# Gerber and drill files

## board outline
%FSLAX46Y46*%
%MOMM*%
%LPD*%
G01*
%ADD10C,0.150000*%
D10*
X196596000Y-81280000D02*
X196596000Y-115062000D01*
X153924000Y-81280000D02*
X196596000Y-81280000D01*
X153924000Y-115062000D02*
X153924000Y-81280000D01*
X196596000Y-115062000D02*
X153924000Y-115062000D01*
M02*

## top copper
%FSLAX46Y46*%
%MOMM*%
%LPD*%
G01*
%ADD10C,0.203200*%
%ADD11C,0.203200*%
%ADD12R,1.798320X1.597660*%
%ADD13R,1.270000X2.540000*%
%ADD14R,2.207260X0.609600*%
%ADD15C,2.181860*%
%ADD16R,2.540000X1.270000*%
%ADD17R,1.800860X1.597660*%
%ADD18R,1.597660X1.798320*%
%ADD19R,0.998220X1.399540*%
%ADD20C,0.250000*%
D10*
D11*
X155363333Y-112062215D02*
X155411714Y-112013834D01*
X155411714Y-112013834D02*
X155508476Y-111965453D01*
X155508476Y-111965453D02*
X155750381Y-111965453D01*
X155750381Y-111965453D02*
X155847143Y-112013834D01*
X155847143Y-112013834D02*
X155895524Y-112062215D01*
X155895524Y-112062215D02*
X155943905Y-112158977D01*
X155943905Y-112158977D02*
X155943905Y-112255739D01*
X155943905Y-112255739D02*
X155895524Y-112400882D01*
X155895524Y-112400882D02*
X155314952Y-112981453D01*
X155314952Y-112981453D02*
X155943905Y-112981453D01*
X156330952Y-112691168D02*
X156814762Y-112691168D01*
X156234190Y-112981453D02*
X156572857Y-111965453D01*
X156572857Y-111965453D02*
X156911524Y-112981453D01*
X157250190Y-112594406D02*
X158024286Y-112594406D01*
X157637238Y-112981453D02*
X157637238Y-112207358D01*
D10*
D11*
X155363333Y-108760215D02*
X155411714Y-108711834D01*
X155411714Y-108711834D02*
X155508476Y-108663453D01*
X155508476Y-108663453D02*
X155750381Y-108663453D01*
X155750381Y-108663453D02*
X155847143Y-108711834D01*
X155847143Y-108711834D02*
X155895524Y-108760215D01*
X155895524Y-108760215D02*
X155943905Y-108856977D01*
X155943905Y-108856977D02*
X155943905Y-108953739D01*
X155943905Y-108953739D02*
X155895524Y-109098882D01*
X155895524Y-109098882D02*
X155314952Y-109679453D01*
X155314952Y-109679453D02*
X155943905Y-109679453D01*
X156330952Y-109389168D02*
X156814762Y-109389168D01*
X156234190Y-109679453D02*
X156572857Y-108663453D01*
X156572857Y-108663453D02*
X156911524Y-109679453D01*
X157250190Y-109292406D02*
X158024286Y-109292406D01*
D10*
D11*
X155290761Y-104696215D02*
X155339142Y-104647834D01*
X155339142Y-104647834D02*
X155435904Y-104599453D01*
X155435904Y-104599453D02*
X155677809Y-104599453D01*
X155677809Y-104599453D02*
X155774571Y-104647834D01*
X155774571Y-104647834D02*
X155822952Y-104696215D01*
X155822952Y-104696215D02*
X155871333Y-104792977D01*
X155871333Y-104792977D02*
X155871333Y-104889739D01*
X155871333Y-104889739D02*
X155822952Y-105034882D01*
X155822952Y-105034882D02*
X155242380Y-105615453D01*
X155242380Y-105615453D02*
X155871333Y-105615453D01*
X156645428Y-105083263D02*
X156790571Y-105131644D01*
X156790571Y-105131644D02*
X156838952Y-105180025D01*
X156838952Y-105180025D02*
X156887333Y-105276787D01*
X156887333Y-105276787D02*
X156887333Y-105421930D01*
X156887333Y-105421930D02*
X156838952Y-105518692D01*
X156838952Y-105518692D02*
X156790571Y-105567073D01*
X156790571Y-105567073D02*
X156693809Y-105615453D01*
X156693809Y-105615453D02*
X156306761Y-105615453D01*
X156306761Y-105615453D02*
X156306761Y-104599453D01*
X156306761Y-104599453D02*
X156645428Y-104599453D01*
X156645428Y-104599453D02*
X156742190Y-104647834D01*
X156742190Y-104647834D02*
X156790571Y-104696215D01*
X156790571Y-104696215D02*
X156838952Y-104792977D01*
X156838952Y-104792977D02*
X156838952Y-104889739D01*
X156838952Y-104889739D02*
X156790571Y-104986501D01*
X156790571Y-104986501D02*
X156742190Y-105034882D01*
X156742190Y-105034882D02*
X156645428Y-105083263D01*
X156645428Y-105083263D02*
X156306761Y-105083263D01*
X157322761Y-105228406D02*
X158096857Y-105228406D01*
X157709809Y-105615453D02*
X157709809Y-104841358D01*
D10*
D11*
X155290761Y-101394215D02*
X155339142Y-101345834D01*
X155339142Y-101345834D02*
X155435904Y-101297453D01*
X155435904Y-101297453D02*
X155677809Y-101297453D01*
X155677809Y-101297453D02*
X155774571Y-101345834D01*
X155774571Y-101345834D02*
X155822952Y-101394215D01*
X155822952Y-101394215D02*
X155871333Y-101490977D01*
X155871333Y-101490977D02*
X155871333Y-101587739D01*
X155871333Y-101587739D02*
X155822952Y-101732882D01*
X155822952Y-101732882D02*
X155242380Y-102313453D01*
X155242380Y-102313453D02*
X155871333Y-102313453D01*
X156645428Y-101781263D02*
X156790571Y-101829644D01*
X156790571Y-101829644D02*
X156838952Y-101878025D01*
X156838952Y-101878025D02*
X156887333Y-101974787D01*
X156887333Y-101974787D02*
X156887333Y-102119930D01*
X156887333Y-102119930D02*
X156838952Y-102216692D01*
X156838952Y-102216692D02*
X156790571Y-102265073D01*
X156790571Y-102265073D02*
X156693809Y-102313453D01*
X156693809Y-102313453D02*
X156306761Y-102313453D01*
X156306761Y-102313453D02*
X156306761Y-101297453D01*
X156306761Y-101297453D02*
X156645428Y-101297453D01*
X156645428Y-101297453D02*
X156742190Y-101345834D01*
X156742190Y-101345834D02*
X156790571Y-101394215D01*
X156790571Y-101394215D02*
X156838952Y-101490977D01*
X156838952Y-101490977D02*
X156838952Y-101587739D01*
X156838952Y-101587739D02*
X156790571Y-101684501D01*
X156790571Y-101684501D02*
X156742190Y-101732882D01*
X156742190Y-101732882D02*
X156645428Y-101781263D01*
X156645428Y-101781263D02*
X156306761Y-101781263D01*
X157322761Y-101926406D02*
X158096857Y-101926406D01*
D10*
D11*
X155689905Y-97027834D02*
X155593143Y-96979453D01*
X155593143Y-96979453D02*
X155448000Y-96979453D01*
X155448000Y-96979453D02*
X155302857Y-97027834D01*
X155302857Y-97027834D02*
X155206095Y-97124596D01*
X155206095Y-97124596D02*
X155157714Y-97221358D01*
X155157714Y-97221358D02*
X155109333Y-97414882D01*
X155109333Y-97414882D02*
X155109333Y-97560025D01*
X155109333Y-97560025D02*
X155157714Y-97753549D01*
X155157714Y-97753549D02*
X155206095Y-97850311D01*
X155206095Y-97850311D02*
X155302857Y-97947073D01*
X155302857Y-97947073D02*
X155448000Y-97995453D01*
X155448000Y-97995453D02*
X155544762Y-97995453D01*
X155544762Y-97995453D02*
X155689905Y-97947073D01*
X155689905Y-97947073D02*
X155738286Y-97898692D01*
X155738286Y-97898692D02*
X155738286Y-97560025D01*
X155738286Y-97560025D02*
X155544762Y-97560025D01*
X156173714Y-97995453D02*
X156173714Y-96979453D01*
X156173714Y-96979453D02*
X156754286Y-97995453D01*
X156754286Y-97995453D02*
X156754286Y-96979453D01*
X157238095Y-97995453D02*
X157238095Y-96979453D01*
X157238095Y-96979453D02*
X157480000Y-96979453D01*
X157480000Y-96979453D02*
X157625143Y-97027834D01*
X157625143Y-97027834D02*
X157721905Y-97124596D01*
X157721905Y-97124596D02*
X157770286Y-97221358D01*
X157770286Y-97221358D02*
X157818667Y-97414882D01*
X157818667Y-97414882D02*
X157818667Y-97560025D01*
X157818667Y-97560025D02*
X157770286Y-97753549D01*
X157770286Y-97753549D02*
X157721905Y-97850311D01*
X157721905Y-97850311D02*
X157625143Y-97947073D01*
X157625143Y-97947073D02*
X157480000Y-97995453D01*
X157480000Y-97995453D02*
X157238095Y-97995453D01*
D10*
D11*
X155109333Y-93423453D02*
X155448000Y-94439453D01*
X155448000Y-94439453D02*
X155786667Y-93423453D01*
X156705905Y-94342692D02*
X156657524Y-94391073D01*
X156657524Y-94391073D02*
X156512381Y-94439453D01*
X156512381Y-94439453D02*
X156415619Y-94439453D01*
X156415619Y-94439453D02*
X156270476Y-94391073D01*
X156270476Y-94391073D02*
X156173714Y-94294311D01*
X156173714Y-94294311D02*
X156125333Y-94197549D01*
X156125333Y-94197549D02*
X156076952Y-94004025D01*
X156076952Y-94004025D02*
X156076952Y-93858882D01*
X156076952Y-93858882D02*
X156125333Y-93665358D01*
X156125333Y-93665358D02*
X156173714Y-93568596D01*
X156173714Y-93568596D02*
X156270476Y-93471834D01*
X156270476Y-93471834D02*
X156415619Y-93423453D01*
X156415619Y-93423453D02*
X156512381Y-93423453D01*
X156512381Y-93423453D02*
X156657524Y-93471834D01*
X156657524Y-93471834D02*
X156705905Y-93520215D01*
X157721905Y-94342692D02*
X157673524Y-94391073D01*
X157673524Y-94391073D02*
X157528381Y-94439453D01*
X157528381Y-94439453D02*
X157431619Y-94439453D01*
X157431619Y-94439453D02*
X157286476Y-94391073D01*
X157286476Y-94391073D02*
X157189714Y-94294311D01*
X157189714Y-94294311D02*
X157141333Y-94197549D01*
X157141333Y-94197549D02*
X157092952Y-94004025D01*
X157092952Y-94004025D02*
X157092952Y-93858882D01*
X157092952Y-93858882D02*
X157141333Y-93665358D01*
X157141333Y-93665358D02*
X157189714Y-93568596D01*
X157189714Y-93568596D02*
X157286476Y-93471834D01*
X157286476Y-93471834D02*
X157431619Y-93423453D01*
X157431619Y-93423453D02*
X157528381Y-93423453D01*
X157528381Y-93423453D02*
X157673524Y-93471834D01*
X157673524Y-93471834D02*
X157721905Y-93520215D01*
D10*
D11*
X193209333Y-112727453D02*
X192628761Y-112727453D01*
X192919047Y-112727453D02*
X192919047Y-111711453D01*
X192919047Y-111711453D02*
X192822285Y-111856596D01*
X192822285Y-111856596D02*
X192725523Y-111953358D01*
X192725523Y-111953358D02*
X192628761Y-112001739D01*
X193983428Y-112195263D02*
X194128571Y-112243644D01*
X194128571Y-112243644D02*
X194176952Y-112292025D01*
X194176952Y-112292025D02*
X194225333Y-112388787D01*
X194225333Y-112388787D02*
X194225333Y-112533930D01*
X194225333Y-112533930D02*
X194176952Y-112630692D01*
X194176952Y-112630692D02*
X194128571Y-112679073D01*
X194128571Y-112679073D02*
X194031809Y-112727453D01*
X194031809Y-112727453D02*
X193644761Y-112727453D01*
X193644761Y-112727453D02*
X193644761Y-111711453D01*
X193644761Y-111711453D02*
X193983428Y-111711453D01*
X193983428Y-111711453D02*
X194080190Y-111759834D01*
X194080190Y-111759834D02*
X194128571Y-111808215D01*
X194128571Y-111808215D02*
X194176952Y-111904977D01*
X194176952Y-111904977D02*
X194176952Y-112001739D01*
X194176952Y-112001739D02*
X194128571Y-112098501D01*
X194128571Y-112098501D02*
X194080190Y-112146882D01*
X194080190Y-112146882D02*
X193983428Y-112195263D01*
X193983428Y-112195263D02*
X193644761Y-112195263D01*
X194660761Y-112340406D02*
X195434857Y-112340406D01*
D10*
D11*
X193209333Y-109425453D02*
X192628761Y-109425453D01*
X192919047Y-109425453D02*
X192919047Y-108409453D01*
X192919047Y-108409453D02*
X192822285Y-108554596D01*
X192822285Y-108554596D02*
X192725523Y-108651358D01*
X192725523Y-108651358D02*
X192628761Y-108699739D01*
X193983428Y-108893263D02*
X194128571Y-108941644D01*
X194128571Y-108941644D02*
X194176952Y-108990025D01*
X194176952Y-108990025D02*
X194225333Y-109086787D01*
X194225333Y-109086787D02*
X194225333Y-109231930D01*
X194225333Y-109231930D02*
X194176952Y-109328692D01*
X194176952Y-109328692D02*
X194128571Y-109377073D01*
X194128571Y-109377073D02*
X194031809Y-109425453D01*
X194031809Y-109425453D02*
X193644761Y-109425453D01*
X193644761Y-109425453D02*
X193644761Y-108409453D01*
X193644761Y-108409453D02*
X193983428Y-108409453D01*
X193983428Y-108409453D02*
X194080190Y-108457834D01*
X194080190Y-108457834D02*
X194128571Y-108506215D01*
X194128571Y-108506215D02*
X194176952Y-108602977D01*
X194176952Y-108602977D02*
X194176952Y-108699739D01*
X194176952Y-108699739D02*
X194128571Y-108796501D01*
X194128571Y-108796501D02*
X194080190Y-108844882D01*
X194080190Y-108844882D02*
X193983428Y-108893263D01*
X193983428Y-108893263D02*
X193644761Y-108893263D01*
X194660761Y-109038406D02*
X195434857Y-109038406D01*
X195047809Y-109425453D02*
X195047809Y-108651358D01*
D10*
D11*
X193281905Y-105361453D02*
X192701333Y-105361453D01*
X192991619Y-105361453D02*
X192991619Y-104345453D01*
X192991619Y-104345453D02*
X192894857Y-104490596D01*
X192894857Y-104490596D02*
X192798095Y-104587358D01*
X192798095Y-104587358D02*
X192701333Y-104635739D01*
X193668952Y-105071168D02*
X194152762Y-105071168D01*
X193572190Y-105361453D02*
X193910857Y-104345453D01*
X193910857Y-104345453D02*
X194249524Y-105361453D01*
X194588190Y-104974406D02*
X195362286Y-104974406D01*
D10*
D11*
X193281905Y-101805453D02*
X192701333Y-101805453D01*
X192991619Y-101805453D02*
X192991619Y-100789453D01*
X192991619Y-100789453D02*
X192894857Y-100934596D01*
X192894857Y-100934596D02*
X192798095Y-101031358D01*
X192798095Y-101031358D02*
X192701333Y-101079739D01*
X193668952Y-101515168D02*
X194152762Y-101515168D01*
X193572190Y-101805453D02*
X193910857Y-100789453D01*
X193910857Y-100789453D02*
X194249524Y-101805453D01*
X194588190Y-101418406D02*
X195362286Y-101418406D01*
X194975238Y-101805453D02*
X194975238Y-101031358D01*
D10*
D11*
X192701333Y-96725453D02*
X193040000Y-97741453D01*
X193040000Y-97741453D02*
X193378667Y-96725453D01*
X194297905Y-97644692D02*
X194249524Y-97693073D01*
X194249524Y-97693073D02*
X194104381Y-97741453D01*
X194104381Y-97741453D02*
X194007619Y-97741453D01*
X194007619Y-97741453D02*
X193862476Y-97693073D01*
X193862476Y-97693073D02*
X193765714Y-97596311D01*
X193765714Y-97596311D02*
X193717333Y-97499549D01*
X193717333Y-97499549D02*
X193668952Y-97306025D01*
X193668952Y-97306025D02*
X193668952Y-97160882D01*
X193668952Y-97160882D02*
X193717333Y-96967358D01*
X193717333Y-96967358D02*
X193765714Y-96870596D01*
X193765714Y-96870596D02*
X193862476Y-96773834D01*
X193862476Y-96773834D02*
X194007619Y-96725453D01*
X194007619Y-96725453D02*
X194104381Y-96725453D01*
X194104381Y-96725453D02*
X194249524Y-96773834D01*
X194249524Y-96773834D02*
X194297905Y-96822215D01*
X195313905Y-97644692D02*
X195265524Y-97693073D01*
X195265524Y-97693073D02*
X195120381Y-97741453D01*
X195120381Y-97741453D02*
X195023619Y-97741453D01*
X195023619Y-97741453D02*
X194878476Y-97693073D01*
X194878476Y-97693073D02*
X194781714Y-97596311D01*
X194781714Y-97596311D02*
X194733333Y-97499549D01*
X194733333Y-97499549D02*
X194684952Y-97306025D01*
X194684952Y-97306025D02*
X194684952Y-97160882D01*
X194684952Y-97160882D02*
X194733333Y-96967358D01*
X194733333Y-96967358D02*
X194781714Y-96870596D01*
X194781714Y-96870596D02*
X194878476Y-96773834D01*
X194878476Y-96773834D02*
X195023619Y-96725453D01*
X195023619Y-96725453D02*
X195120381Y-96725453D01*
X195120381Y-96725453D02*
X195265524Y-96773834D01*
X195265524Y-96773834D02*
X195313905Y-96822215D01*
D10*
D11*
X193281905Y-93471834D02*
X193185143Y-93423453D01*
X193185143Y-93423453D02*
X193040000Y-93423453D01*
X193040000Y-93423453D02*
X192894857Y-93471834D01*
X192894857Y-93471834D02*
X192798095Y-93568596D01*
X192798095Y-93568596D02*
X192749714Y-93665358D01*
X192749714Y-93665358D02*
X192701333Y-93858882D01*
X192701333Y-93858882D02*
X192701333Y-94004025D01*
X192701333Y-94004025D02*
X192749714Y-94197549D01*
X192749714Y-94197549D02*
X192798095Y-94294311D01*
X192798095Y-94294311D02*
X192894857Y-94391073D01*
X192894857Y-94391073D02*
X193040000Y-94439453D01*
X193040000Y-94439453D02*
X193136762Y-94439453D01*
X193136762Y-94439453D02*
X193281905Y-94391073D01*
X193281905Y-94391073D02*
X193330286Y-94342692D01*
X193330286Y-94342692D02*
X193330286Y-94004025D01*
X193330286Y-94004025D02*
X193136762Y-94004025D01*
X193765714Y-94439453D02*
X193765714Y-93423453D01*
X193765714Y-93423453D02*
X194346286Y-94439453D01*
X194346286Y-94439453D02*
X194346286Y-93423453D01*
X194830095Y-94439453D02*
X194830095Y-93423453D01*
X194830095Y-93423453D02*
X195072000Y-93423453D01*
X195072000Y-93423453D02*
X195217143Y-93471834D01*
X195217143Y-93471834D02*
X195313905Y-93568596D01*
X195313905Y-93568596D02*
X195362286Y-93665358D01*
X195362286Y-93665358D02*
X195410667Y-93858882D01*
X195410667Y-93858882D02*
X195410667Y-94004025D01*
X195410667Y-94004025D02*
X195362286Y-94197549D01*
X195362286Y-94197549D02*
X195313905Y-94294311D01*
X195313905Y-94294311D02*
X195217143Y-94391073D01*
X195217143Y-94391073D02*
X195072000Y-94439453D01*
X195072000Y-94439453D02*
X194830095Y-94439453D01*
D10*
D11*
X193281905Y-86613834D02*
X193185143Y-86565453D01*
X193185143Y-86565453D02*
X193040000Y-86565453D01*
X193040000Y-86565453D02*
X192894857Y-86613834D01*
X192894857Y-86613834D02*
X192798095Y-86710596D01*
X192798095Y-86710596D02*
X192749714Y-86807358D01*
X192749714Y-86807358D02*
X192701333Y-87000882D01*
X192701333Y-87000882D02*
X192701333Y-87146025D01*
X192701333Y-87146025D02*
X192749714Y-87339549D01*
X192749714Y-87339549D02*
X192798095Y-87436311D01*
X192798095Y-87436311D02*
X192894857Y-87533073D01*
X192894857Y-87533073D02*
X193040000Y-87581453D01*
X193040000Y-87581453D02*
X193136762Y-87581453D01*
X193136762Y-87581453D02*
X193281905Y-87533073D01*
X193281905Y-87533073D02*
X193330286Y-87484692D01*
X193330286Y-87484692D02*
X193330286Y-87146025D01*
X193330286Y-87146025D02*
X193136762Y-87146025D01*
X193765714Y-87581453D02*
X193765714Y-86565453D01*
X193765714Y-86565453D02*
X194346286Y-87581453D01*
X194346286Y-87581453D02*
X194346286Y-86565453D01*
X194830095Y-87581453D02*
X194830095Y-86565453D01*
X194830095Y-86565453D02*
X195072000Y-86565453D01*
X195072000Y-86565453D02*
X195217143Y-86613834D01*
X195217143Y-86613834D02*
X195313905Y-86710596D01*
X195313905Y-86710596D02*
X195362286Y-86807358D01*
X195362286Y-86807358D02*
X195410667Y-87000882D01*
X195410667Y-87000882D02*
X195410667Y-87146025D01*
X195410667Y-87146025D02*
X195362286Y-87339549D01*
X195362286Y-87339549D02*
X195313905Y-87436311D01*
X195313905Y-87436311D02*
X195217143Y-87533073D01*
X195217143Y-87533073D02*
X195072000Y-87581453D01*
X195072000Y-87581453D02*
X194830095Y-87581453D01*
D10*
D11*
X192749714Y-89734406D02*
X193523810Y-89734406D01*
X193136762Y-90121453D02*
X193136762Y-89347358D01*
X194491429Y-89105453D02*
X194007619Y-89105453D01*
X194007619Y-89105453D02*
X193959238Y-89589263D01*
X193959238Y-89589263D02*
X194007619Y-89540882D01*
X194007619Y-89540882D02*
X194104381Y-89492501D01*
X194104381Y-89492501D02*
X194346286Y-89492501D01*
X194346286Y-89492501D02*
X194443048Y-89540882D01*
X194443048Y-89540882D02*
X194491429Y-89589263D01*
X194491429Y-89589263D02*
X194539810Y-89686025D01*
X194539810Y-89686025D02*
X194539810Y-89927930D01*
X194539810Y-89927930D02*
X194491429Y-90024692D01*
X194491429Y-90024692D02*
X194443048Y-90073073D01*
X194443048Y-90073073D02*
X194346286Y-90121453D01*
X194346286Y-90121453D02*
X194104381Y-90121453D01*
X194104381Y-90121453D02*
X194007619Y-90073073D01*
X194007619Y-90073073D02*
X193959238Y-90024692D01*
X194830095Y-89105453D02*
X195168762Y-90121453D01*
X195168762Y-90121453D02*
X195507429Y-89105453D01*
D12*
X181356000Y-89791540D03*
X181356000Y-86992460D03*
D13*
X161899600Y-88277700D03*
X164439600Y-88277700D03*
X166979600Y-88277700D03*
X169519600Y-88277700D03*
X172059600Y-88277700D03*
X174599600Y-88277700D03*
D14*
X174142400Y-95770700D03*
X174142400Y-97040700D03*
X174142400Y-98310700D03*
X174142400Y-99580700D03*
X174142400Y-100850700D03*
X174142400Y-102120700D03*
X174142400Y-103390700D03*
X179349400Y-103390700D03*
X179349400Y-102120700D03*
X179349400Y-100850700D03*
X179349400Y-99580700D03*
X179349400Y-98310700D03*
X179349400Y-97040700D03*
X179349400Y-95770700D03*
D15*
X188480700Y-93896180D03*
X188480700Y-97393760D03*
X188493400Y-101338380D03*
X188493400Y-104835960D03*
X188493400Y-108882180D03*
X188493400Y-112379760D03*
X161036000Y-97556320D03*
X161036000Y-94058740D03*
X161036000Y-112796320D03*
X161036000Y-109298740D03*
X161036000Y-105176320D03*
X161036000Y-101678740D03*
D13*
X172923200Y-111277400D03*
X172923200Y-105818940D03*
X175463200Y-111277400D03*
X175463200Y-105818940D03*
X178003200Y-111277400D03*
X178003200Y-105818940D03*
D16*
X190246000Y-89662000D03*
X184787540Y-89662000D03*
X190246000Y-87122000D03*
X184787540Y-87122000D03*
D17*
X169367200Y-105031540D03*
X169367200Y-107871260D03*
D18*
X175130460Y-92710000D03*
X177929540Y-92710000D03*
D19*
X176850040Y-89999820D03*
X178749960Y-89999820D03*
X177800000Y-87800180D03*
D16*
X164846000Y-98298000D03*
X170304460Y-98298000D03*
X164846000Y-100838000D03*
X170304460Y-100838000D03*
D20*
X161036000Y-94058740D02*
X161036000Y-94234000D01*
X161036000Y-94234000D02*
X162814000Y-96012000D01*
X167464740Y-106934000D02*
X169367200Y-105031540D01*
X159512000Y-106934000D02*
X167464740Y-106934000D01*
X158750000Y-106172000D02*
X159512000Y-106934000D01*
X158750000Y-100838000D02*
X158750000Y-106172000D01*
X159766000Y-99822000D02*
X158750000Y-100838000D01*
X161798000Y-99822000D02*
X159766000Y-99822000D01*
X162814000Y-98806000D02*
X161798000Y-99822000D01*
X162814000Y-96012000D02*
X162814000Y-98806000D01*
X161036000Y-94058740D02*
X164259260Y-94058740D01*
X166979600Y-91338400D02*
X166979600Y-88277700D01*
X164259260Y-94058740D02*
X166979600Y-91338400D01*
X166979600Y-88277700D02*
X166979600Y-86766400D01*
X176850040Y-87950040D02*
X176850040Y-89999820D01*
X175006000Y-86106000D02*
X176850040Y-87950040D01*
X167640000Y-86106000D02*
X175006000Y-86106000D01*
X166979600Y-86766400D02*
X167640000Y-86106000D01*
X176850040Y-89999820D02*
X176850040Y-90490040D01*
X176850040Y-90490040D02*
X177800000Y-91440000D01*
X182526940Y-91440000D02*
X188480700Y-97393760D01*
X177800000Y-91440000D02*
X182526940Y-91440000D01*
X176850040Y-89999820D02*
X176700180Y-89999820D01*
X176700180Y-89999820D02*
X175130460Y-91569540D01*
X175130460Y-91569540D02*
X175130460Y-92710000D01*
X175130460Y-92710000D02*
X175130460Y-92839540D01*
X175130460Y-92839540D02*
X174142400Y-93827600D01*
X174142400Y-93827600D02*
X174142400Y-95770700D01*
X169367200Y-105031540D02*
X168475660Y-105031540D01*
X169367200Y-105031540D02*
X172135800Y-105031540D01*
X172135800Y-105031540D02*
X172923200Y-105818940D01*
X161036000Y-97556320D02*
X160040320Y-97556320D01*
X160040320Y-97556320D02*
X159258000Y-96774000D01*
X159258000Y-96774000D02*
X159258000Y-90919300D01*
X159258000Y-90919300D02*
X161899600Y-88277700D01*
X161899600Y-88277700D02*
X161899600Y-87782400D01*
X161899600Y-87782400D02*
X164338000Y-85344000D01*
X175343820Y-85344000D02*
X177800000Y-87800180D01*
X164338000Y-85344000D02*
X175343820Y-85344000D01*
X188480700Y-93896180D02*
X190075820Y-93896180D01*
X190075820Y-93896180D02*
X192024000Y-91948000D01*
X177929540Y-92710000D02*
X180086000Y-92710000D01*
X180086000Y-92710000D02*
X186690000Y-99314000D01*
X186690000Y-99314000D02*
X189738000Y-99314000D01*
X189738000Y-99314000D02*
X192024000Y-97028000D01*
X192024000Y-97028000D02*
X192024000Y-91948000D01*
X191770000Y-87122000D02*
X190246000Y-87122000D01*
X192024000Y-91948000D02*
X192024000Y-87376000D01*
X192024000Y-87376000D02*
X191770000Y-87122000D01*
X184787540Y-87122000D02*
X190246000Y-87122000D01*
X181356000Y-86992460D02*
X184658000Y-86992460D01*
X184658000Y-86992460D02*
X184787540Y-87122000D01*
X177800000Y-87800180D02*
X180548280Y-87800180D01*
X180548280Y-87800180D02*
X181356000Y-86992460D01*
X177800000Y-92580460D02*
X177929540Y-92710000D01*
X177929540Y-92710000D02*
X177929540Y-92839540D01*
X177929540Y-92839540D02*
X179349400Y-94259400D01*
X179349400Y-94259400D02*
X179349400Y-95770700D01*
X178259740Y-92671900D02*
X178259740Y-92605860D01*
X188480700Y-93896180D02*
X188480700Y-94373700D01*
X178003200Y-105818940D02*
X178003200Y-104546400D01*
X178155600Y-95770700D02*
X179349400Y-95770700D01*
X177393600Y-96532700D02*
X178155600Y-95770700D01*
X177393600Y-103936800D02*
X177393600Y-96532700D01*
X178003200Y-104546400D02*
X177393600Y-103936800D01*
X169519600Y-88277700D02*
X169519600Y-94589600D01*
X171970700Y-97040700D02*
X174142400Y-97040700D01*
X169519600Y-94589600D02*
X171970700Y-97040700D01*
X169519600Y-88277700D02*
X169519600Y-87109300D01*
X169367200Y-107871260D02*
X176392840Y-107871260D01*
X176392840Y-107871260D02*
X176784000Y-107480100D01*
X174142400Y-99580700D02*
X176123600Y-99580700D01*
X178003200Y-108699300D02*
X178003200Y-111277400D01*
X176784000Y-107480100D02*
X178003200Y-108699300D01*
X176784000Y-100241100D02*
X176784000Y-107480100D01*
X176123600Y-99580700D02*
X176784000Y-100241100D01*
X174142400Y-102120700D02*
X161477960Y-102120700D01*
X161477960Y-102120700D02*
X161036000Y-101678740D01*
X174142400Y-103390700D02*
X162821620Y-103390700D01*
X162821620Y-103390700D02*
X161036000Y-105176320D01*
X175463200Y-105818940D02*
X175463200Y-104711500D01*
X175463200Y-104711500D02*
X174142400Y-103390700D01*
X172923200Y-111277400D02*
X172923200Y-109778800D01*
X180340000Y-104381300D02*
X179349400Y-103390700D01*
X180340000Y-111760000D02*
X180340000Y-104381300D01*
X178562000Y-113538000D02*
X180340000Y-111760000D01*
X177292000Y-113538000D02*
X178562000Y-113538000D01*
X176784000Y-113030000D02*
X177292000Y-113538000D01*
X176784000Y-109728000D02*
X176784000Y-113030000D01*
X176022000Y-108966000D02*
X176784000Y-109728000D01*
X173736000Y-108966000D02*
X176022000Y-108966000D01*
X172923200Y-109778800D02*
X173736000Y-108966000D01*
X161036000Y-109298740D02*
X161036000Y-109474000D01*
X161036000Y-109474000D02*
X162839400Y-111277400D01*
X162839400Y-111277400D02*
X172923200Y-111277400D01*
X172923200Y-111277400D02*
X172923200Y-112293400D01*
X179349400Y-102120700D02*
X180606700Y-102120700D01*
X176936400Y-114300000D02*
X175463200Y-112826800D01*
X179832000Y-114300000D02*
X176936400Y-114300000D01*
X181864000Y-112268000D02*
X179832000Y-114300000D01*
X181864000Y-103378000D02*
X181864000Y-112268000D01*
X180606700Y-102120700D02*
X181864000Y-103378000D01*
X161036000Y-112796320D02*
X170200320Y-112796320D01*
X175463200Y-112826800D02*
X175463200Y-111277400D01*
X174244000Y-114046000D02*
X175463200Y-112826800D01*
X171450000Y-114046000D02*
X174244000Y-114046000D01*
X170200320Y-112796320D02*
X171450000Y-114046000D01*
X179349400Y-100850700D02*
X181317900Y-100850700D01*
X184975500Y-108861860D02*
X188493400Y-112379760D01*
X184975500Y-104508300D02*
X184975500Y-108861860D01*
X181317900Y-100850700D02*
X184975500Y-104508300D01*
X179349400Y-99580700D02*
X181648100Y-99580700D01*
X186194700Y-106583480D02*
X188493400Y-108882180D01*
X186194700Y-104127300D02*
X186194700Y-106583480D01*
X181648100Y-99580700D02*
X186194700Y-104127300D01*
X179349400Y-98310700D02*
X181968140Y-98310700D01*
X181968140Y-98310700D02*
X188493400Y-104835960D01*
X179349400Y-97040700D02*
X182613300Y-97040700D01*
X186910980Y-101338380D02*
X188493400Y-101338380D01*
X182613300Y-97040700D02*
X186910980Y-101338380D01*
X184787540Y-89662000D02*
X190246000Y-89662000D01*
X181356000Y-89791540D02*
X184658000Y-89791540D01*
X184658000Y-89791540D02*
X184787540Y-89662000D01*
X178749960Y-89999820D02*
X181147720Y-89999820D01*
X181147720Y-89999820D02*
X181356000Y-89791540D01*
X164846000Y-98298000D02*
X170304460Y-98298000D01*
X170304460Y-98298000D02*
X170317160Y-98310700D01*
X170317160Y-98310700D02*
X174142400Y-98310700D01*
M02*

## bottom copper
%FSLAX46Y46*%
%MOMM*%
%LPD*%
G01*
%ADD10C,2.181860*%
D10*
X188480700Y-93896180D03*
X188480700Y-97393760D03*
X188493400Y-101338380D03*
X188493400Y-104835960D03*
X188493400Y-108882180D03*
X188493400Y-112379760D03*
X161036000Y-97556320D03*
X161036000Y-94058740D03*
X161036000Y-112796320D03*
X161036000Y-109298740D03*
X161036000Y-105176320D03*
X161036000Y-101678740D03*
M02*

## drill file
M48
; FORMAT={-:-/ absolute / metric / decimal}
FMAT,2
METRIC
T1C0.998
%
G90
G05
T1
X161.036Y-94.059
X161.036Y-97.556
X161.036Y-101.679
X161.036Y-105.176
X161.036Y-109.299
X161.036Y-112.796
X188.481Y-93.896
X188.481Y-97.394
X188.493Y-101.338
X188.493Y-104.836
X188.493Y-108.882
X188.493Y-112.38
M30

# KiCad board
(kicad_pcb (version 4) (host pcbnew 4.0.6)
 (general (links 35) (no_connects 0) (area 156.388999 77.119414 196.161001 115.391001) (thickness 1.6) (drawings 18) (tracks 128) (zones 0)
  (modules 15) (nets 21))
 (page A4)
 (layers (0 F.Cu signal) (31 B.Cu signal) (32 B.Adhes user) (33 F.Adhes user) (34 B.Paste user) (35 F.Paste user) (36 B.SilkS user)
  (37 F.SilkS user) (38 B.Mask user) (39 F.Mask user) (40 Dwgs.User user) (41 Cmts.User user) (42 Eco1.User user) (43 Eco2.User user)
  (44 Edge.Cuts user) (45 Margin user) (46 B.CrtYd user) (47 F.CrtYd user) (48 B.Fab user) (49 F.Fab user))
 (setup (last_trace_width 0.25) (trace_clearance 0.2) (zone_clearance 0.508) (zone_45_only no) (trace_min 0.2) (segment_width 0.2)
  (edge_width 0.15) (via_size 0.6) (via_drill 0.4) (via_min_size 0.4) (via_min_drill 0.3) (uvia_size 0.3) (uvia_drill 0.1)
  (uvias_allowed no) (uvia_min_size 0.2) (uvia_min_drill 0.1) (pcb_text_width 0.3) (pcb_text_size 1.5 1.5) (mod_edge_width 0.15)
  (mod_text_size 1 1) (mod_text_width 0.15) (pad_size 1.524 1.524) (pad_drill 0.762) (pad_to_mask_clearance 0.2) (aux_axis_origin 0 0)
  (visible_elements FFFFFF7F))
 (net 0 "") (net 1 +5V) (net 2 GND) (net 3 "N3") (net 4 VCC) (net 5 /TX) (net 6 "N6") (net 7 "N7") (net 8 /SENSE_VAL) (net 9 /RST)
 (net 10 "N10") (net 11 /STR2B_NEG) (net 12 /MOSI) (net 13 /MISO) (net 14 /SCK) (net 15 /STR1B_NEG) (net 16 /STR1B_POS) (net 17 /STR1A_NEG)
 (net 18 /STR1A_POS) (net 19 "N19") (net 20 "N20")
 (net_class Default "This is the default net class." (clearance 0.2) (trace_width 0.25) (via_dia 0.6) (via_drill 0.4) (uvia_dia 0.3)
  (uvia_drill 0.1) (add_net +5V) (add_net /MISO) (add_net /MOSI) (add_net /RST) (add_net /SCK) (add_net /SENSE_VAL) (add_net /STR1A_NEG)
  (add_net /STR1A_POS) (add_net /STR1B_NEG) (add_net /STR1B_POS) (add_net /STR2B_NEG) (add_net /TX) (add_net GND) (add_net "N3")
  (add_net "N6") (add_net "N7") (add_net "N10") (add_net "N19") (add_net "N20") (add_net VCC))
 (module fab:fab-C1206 (layer F.Cu) (at 181.356 88.392 90)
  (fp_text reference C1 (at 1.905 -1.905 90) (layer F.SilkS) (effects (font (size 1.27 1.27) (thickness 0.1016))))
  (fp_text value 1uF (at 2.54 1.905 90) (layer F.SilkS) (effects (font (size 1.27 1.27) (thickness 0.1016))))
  (pad 1 smd rect (at -1.39954 0 90) (size 1.59766 1.79832) (layers F.Cu F.Paste F.Mask) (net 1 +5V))
  (pad 2 smd rect (at 1.39954 0 90) (size 1.59766 1.79832) (layers F.Cu F.Paste F.Mask) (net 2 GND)))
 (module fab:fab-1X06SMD (layer F.Cu) (at 168.2496 88.2777 90)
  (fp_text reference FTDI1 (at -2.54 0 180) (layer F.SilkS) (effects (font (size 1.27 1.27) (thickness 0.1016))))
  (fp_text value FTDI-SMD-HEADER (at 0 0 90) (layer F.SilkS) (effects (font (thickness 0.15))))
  (pad 1 smd rect (at 0 -6.35 90) (size 2.54 1.27) (layers F.Cu F.Paste F.Mask) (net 2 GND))
  (pad 2 smd rect (at 0 -3.81 90) (size 2.54 1.27) (layers F.Cu F.Paste F.Mask) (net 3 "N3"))
  (pad 3 smd rect (at 0 -1.27 90) (size 2.54 1.27) (layers F.Cu F.Paste F.Mask) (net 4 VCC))
  (pad 4 smd rect (at 0 1.27 90) (size 2.54 1.27) (layers F.Cu F.Paste F.Mask) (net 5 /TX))
  (pad 5 smd rect (at 0 3.81 90) (size 2.54 1.27) (layers F.Cu F.Paste F.Mask) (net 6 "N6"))
  (pad 6 smd rect (at 0 6.35 90) (size 2.54 1.27) (layers F.Cu F.Paste F.Mask) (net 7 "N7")))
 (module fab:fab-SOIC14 (layer F.Cu) (at 176.7459 99.5807 270)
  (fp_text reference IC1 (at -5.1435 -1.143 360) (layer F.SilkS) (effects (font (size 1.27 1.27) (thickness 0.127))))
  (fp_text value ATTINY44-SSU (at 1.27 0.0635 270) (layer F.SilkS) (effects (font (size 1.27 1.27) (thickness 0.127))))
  (pad 1 smd rect (at -3.81 2.6035 270) (size 0.6096 2.20726) (layers F.Cu F.Paste F.Mask) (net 4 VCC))
  (pad 2 smd rect (at -2.54 2.6035 270) (size 0.6096 2.20726) (layers F.Cu F.Paste F.Mask) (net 5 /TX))
  (pad 3 smd rect (at -1.27 2.6035 270) (size 0.6096 2.20726) (layers F.Cu F.Paste F.Mask) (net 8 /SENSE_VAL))
  (pad 4 smd rect (at 0 2.6035 270) (size 0.6096 2.20726) (layers F.Cu F.Paste F.Mask) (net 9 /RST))
  (pad 5 smd rect (at 1.27 2.6035 270) (size 0.6096 2.20726) (layers F.Cu F.Paste F.Mask) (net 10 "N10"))
  (pad 6 smd rect (at 2.54 2.6035 270) (size 0.6096 2.20726) (layers F.Cu F.Paste F.Mask) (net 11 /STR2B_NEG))
  (pad 7 smd rect (at 3.81 2.6035 270) (size 0.6096 2.20726) (layers F.Cu F.Paste F.Mask) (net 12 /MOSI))
  (pad 8 smd rect (at 3.81 -2.6035 270) (size 0.6096 2.20726) (layers F.Cu F.Paste F.Mask) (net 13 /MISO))
  (pad 9 smd rect (at 2.54 -2.6035 270) (size 0.6096 2.20726) (layers F.Cu F.Paste F.Mask) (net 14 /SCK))
  (pad 10 smd rect (at 1.27 -2.6035 270) (size 0.6096 2.20726) (layers F.Cu F.Paste F.Mask) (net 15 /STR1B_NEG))
  (pad 11 smd rect (at 0 -2.6035 270) (size 0.6096 2.20726) (layers F.Cu F.Paste F.Mask) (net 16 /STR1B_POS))
  (pad 12 smd rect (at -1.27 -2.6035 270) (size 0.6096 2.20726) (layers F.Cu F.Paste F.Mask) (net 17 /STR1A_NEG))
  (pad 13 smd rect (at -2.54 -2.6035 270) (size 0.6096 2.20726) (layers F.Cu F.Paste F.Mask) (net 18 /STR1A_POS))
  (pad 14 smd rect (at -3.81 -2.6035 270) (size 0.6096 2.20726) (layers F.Cu F.Paste F.Mask) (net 2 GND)))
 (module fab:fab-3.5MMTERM (layer F.Cu) (at 188.4807 95.6945 90)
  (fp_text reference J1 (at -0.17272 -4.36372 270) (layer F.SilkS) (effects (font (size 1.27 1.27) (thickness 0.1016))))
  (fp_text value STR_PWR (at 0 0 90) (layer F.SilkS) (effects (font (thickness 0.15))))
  (pad 1 thru_hole circle (at 1.79832 0 90) (size 2.18186 2.18186) (drill 0.99822) (layers *.Cu F.Paste F.SilkS F.Mask) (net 2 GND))
  (pad 2 thru_hole circle (at -1.69926 0 90) (size 2.18186 2.18186) (drill 0.99822) (layers *.Cu F.Paste F.SilkS F.Mask) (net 4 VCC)))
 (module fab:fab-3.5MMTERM (layer F.Cu) (at 188.4934 103.1367 90)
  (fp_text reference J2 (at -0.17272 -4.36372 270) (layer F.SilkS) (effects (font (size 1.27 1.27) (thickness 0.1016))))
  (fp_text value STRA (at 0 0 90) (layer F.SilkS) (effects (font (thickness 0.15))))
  (pad 1 thru_hole circle (at 1.79832 0 90) (size 2.18186 2.18186) (drill 0.99822) (layers *.Cu F.Paste F.SilkS F.Mask) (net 18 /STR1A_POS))
  (pad 2 thru_hole circle (at -1.69926 0 90) (size 2.18186 2.18186) (drill 0.99822) (layers *.Cu F.Paste F.SilkS F.Mask) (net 17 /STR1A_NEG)))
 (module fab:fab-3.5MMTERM (layer F.Cu) (at 188.4934 110.6805 90)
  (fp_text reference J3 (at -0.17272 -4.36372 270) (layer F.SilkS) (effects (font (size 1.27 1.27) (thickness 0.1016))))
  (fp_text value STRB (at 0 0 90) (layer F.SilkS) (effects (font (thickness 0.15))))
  (pad 1 thru_hole circle (at 1.79832 0 90) (size 2.18186 2.18186) (drill 0.99822) (layers *.Cu F.Paste F.SilkS F.Mask) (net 16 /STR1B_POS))
  (pad 2 thru_hole circle (at -1.69926 0 90) (size 2.18186 2.18186) (drill 0.99822) (layers *.Cu F.Paste F.SilkS F.Mask) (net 15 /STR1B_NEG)))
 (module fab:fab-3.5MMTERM (layer F.Cu) (at 161.036 95.758 270)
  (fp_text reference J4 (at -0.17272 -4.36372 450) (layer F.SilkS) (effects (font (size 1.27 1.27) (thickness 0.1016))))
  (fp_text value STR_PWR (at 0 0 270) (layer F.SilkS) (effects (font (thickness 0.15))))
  (pad 1 thru_hole circle (at 1.79832 0 270) (size 2.18186 2.18186) (drill 0.99822) (layers *.Cu F.Paste F.SilkS F.Mask) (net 2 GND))
  (pad 2 thru_hole circle (at -1.69926 0 270) (size 2.18186 2.18186) (drill 0.99822) (layers *.Cu F.Paste F.SilkS F.Mask) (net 4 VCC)))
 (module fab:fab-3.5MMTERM (layer F.Cu) (at 161.036 110.998 270)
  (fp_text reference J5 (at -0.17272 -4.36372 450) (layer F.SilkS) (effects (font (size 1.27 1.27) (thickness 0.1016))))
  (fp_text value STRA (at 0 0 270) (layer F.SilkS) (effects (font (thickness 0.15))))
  (pad 1 thru_hole circle (at 1.79832 0 270) (size 2.18186 2.18186) (drill 0.99822) (layers *.Cu F.Paste F.SilkS F.Mask) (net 14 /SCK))
  (pad 2 thru_hole circle (at -1.69926 0 270) (size 2.18186 2.18186) (drill 0.99822) (layers *.Cu F.Paste F.SilkS F.Mask) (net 13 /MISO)))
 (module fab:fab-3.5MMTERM (layer F.Cu) (at 161.036 103.378 270)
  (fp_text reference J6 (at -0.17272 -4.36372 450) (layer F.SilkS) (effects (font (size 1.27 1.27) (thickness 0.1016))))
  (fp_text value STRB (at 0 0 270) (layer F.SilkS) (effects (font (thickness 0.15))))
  (pad 1 thru_hole circle (at 1.79832 0 270) (size 2.18186 2.18186) (drill 0.99822) (layers *.Cu F.Paste F.SilkS F.Mask) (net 12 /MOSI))
  (pad 2 thru_hole circle (at -1.69926 0 270) (size 2.18186 2.18186) (drill 0.99822) (layers *.Cu F.Paste F.SilkS F.Mask)
   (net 11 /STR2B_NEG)))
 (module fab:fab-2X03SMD (layer F.Cu) (at 175.4632 108.7374 90)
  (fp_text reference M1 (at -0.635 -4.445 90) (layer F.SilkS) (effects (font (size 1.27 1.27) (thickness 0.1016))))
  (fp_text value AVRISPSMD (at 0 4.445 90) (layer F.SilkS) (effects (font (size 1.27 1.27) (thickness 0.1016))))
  (pad 1 smd rect (at -2.54 -2.54 90) (size 2.54 1.27) (layers F.Cu F.Paste F.Mask) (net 13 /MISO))
  (pad 2 smd rect (at 2.91846 -2.54 90) (size 2.54 1.27) (layers F.Cu F.Paste F.Mask) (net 4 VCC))
  (pad 3 smd rect (at -2.54 0 90) (size 2.54 1.27) (layers F.Cu F.Paste F.Mask) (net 14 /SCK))
  (pad 4 smd rect (at 2.91846 0 90) (size 2.54 1.27) (layers F.Cu F.Paste F.Mask) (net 12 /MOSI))
  (pad 5 smd rect (at -2.54 2.54 90) (size 2.54 1.27) (layers F.Cu F.Paste F.Mask) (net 9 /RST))
  (pad 6 smd rect (at 2.91846 2.54 90) (size 2.54 1.27) (layers F.Cu F.Paste F.Mask) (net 2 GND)))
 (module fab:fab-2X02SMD (layer F.Cu) (at 187.706 88.392 180)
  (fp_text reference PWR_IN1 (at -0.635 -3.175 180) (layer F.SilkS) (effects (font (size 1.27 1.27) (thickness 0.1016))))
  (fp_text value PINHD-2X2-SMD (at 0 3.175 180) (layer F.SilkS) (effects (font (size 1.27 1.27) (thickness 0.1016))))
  (pad 1 smd rect (at -2.54 -1.27 180) (size 2.54 1.27) (layers F.Cu F.Paste F.Mask) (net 1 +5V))
  (pad 2 smd rect (at 2.91846 -1.27 180) (size 2.54 1.27) (layers F.Cu F.Paste F.Mask) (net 1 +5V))
  (pad 3 smd rect (at -2.54 1.27 180) (size 2.54 1.27) (layers F.Cu F.Paste F.Mask) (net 2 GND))
  (pad 4 smd rect (at 2.91846 1.27 180) (size 2.54 1.27) (layers F.Cu F.Paste F.Mask) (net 2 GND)))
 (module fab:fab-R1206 (layer F.Cu) (at 169.3672 106.4514 270)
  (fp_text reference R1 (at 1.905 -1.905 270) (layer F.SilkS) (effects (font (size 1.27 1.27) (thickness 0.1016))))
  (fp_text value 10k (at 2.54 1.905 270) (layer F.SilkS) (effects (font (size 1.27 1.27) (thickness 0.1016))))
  (pad 1 smd rect (at -1.41986 0 270) (size 1.59766 1.80086) (layers F.Cu F.Paste F.Mask) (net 4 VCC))
  (pad 2 smd rect (at 1.41986 0 270) (size 1.59766 1.80086) (layers F.Cu F.Paste F.Mask) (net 9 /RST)))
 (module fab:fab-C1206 (layer F.Cu) (at 176.53 92.71)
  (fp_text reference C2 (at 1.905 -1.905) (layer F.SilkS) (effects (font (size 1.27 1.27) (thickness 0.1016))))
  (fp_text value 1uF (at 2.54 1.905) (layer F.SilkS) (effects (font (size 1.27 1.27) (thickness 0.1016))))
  (pad 1 smd rect (at -1.39954 0) (size 1.59766 1.79832) (layers F.Cu F.Paste F.Mask) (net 4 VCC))
  (pad 2 smd rect (at 1.39954 0) (size 1.59766 1.79832) (layers F.Cu F.Paste F.Mask) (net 2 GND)))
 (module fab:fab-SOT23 (layer F.Cu) (at 177.8 88.9)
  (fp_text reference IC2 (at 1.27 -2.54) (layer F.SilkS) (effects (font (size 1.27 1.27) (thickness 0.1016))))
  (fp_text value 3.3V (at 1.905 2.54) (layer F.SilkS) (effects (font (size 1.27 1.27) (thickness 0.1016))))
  (pad 1 smd rect (at -0.94996 1.09982) (size 0.99822 1.39954) (layers F.Cu F.Paste F.Mask) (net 4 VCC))
  (pad 2 smd rect (at 0.94996 1.09982) (size 0.99822 1.39954) (layers F.Cu F.Paste F.Mask) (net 1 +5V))
  (pad 3 smd rect (at 0 -1.09982) (size 0.99822 1.39954) (layers F.Cu F.Paste F.Mask) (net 2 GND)))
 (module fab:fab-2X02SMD (layer F.Cu) (at 167.386 99.568)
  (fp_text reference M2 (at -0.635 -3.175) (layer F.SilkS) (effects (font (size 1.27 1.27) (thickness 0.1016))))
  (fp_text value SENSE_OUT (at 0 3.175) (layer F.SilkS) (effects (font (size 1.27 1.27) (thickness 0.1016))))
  (pad 1 smd rect (at -2.54 -1.27) (size 2.54 1.27) (layers F.Cu F.Paste F.Mask) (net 8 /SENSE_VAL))
  (pad 2 smd rect (at 2.91846 -1.27) (size 2.54 1.27) (layers F.Cu F.Paste F.Mask) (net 8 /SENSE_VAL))
  (pad 3 smd rect (at -2.54 1.27) (size 2.54 1.27) (layers F.Cu F.Paste F.Mask) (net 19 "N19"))
  (pad 4 smd rect (at 2.91846 1.27) (size 2.54 1.27) (layers F.Cu F.Paste F.Mask) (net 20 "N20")))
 (gr_line (start 196.596 81.28) (end 196.596 115.062) (angle 90) (layer Edge.Cuts) (width 0.15))
 (gr_line (start 153.924 81.28) (end 196.596 81.28) (angle 90) (layer Edge.Cuts) (width 0.15))
 (gr_line (start 153.924 115.062) (end 153.924 81.28) (angle 90) (layer Edge.Cuts) (width 0.15))
 (gr_line (start 196.596 115.062) (end 153.924 115.062) (angle 90) (layer Edge.Cuts) (width 0.15))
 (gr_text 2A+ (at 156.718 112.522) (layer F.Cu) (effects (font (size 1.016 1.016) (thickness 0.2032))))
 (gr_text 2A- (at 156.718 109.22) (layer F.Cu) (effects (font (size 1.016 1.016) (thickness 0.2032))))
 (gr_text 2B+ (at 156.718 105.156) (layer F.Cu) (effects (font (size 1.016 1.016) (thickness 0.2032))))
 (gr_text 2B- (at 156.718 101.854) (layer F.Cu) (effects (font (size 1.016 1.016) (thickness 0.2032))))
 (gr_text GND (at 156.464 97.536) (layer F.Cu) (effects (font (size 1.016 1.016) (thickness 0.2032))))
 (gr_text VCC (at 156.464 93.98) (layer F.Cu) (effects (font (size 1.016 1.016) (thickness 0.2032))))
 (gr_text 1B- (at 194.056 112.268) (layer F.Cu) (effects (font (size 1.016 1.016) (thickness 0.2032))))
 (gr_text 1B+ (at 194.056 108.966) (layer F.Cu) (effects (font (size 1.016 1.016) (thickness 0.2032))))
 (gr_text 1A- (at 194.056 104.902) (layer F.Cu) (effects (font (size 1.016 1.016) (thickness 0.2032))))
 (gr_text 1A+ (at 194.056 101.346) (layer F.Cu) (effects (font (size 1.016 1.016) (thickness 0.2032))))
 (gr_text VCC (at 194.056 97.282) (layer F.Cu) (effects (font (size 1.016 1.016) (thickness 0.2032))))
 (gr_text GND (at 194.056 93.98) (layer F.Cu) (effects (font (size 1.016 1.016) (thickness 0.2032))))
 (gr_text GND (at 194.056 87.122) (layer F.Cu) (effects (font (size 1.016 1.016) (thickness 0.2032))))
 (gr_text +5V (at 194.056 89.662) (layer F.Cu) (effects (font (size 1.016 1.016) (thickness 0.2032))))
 (segment (start 161.036 94.05874) (end 161.036 94.234) (width 0.25) (layer F.Cu) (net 4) (status C00000))
 (segment (start 161.036 94.234) (end 162.814 96.012) (width 0.25) (layer F.Cu) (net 4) (status 400000))
 (segment (start 167.46474 106.934) (end 169.3672 105.03154) (width 0.25) (layer F.Cu) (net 4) (status 800000))
 (segment (start 159.512 106.934) (end 167.46474 106.934) (width 0.25) (layer F.Cu) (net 4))
 (segment (start 158.75 106.172) (end 159.512 106.934) (width 0.25) (layer F.Cu) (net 4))
 (segment (start 158.75 100.838) (end 158.75 106.172) (width 0.25) (layer F.Cu) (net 4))
 (segment (start 159.766 99.822) (end 158.75 100.838) (width 0.25) (layer F.Cu) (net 4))
 (segment (start 161.798 99.822) (end 159.766 99.822) (width 0.25) (layer F.Cu) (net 4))
 (segment (start 162.814 98.806) (end 161.798 99.822) (width 0.25) (layer F.Cu) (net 4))
 (segment (start 162.814 96.012) (end 162.814 98.806) (width 0.25) (layer F.Cu) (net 4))
 (segment (start 161.036 94.05874) (end 164.25926 94.05874) (width 0.25) (layer F.Cu) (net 4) (status 400000))
 (segment (start 166.9796 91.3384) (end 166.9796 88.2777) (width 0.25) (layer F.Cu) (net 4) (status 800000))
 (segment (start 164.25926 94.05874) (end 166.9796 91.3384) (width 0.25) (layer F.Cu) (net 4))
 (segment (start 166.9796 88.2777) (end 166.9796 86.7664) (width 0.25) (layer F.Cu) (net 4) (status 400000))
 (segment (start 176.85004 87.95004) (end 176.85004 89.99982) (width 0.25) (layer F.Cu) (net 4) (status 800000))
 (segment (start 175.006 86.106) (end 176.85004 87.95004) (width 0.25) (layer F.Cu) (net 4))
 (segment (start 167.64 86.106) (end 175.006 86.106) (width 0.25) (layer F.Cu) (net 4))
 (segment (start 166.9796 86.7664) (end 167.64 86.106) (width 0.25) (layer F.Cu) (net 4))
 (segment (start 176.85004 89.99982) (end 176.85004 90.49004) (width 0.25) (layer F.Cu) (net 4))
 (segment (start 176.85004 90.49004) (end 177.8 91.44) (width 0.25) (layer F.Cu) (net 4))
 (segment (start 182.52694 91.44) (end 188.4807 97.39376) (width 0.25) (layer F.Cu) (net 4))
 (segment (start 177.8 91.44) (end 182.52694 91.44) (width 0.25) (layer F.Cu) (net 4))
 (segment (start 176.85004 89.99982) (end 176.70018 89.99982) (width 0.25) (layer F.Cu) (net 4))
 (segment (start 176.70018 89.99982) (end 175.13046 91.56954) (width 0.25) (layer F.Cu) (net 4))
 (segment (start 175.13046 91.56954) (end 175.13046 92.71) (width 0.25) (layer F.Cu) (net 4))
 (segment (start 175.13046 92.71) (end 175.13046 92.83954) (width 0.25) (layer F.Cu) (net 4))
 (segment (start 175.13046 92.83954) (end 174.1424 93.8276) (width 0.25) (layer F.Cu) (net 4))
 (segment (start 174.1424 93.8276) (end 174.1424 95.7707) (width 0.25) (layer F.Cu) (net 4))
 (segment (start 169.3672 105.03154) (end 168.47566 105.03154) (width 0.25) (layer F.Cu) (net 4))
 (segment (start 169.3672 105.03154) (end 172.1358 105.03154) (width 0.25) (layer F.Cu) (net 4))
 (segment (start 172.1358 105.03154) (end 172.9232 105.81894) (width 0.25) (layer F.Cu) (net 4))
 (segment (start 161.036 97.55632) (end 160.04032 97.55632) (width 0.25) (layer F.Cu) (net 2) (status C00000))
 (segment (start 160.04032 97.55632) (end 159.258 96.774) (width 0.25) (layer F.Cu) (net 2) (status 400000))
 (segment (start 159.258 96.774) (end 159.258 90.9193) (width 0.25) (layer F.Cu) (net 2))
 (segment (start 159.258 90.9193) (end 161.8996 88.2777) (width 0.25) (layer F.Cu) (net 2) (status 800000))
 (segment (start 161.8996 88.2777) (end 161.8996 87.7824) (width 0.25) (layer F.Cu) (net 2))
 (segment (start 161.8996 87.7824) (end 164.338 85.344) (width 0.25) (layer F.Cu) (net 2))
 (segment (start 175.34382 85.344) (end 177.8 87.80018) (width 0.25) (layer F.Cu) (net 2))
 (segment (start 164.338 85.344) (end 175.34382 85.344) (width 0.25) (layer F.Cu) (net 2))
 (segment (start 188.4807 93.89618) (end 190.07582 93.89618) (width 0.25) (layer F.Cu) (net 2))
 (segment (start 190.07582 93.89618) (end 192.024 91.948) (width 0.25) (layer F.Cu) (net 2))
 (segment (start 177.92954 92.71) (end 180.086 92.71) (width 0.25) (layer F.Cu) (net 2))
 (segment (start 180.086 92.71) (end 186.69 99.314) (width 0.25) (layer F.Cu) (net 2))
 (segment (start 186.69 99.314) (end 189.738 99.314) (width 0.25) (layer F.Cu) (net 2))
 (segment (start 189.738 99.314) (end 192.024 97.028) (width 0.25) (layer F.Cu) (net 2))
 (segment (start 192.024 97.028) (end 192.024 91.948) (width 0.25) (layer F.Cu) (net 2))
 (segment (start 191.77 87.122) (end 190.246 87.122) (width 0.25) (layer F.Cu) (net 2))
 (segment (start 192.024 91.948) (end 192.024 87.376) (width 0.25) (layer F.Cu) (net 2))
 (segment (start 192.024 87.376) (end 191.77 87.122) (width 0.25) (layer F.Cu) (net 2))
 (segment (start 184.78754 87.122) (end 190.246 87.122) (width 0.25) (layer F.Cu) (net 2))
 (segment (start 181.356 86.99246) (end 184.658 86.99246) (width 0.25) (layer F.Cu) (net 2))
 (segment (start 184.658 86.99246) (end 184.78754 87.122) (width 0.25) (layer F.Cu) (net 2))
 (segment (start 177.8 87.80018) (end 180.54828 87.80018) (width 0.25) (layer F.Cu) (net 2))
 (segment (start 180.54828 87.80018) (end 181.356 86.99246) (width 0.25) (layer F.Cu) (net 2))
 (segment (start 177.8 92.58046) (end 177.92954 92.71) (width 0.25) (layer F.Cu) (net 2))
 (segment (start 177.92954 92.71) (end 177.92954 92.83954) (width 0.25) (layer F.Cu) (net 2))
 (segment (start 177.92954 92.83954) (end 179.3494 94.2594) (width 0.25) (layer F.Cu) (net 2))
 (segment (start 179.3494 94.2594) (end 179.3494 95.7707) (width 0.25) (layer F.Cu) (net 2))
 (segment (start 178.25974 92.6719) (end 178.25974 92.60586) (width 0.25) (layer F.Cu) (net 2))
 (segment (start 188.4807 93.89618) (end 188.4807 94.3737) (width 0.25) (layer F.Cu) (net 2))
 (segment (start 178.0032 105.81894) (end 178.0032 104.5464) (width 0.25) (layer F.Cu) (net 2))
 (segment (start 178.1556 95.7707) (end 179.3494 95.7707) (width 0.25) (layer F.Cu) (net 2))
 (segment (start 177.3936 96.5327) (end 178.1556 95.7707) (width 0.25) (layer F.Cu) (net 2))
 (segment (start 177.3936 103.9368) (end 177.3936 96.5327) (width 0.25) (layer F.Cu) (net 2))
 (segment (start 178.0032 104.5464) (end 177.3936 103.9368) (width 0.25) (layer F.Cu) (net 2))
 (segment (start 169.5196 88.2777) (end 169.5196 94.5896) (width 0.25) (layer F.Cu) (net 5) (status 400000))
 (segment (start 171.9707 97.0407) (end 174.1424 97.0407) (width 0.25) (layer F.Cu) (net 5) (status 800000))
 (segment (start 169.5196 94.5896) (end 171.9707 97.0407) (width 0.25) (layer F.Cu) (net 5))
 (segment (start 169.5196 88.2777) (end 169.5196 87.1093) (width 0.25) (layer F.Cu) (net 5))
 (segment (start 169.3672 107.87126) (end 176.39284 107.87126) (width 0.25) (layer F.Cu) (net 9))
 (segment (start 176.39284 107.87126) (end 176.784 107.4801) (width 0.25) (layer F.Cu) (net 9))
 (segment (start 174.1424 99.5807) (end 176.1236 99.5807) (width 0.25) (layer F.Cu) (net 9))
 (segment (start 178.0032 108.6993) (end 178.0032 111.2774) (width 0.25) (layer F.Cu) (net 9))
 (segment (start 176.784 107.4801) (end 178.0032 108.6993) (width 0.25) (layer F.Cu) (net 9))
 (segment (start 176.784 100.2411) (end 176.784 107.4801) (width 0.25) (layer F.Cu) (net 9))
 (segment (start 176.1236 99.5807) (end 176.784 100.2411) (width 0.25) (layer F.Cu) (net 9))
 (segment (start 174.1424 102.1207) (end 161.47796 102.1207) (width 0.25) (layer F.Cu) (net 11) (status C00000))
 (segment (start 161.47796 102.1207) (end 161.036 101.67874) (width 0.25) (layer F.Cu) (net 11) (status C00000))
 (segment (start 174.1424 103.3907) (end 162.82162 103.3907) (width 0.25) (layer F.Cu) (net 12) (status 400000))
 (segment (start 162.82162 103.3907) (end 161.036 105.17632) (width 0.25) (layer F.Cu) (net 12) (status 800000))
 (segment (start 175.4632 105.81894) (end 175.4632 104.7115) (width 0.25) (layer F.Cu) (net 12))
 (segment (start 175.4632 104.7115) (end 174.1424 103.3907) (width 0.25) (layer F.Cu) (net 12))
 (segment (start 172.9232 111.2774) (end 172.9232 109.7788) (width 0.25) (layer F.Cu) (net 13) (status 400000))
 (segment (start 180.34 104.3813) (end 179.3494 103.3907) (width 0.25) (layer F.Cu) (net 13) (status 800000))
 (segment (start 180.34 111.76) (end 180.34 104.3813) (width 0.25) (layer F.Cu) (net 13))
 (segment (start 178.562 113.538) (end 180.34 111.76) (width 0.25) (layer F.Cu) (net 13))
 (segment (start 177.292 113.538) (end 178.562 113.538) (width 0.25) (layer F.Cu) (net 13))
 (segment (start 176.784 113.03) (end 177.292 113.538) (width 0.25) (layer F.Cu) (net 13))
 (segment (start 176.784 109.728) (end 176.784 113.03) (width 0.25) (layer F.Cu) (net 13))
 (segment (start 176.022 108.966) (end 176.784 109.728) (width 0.25) (layer F.Cu) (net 13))
 (segment (start 173.736 108.966) (end 176.022 108.966) (width 0.25) (layer F.Cu) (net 13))
 (segment (start 172.9232 109.7788) (end 173.736 108.966) (width 0.25) (layer F.Cu) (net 13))
 (segment (start 161.036 109.29874) (end 161.036 109.474) (width 0.25) (layer F.Cu) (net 13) (status C00000))
 (segment (start 161.036 109.474) (end 162.8394 111.2774) (width 0.25) (layer F.Cu) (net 13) (status 400000))
 (segment (start 162.8394 111.2774) (end 172.9232 111.2774) (width 0.25) (layer F.Cu) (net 13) (status 800000))
 (segment (start 172.9232 111.2774) (end 172.9232 112.2934) (width 0.25) (layer F.Cu) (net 13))
 (segment (start 179.3494 102.1207) (end 180.6067 102.1207) (width 0.25) (layer F.Cu) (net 14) (status 400000))
 (segment (start 176.9364 114.3) (end 175.4632 112.8268) (width 0.25) (layer F.Cu) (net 14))
 (segment (start 179.832 114.3) (end 176.9364 114.3) (width 0.25) (layer F.Cu) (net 14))
 (segment (start 181.864 112.268) (end 179.832 114.3) (width 0.25) (layer F.Cu) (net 14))
 (segment (start 181.864 103.378) (end 181.864 112.268) (width 0.25) (layer F.Cu) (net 14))
 (segment (start 180.6067 102.1207) (end 181.864 103.378) (width 0.25) (layer F.Cu) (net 14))
 (segment (start 161.036 112.79632) (end 170.20032 112.79632) (width 0.25) (layer F.Cu) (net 14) (status 400000))
 (segment (start 175.4632 112.8268) (end 175.4632 111.2774) (width 0.25) (layer F.Cu) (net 14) (status 800000))
 (segment (start 174.244 114.046) (end 175.4632 112.8268) (width 0.25) (layer F.Cu) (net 14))
 (segment (start 171.45 114.046) (end 174.244 114.046) (width 0.25) (layer F.Cu) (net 14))
 (segment (start 170.20032 112.79632) (end 171.45 114.046) (width 0.25) (layer F.Cu) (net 14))
 (segment (start 179.3494 100.8507) (end 181.3179 100.8507) (width 0.25) (layer F.Cu) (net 15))
 (segment (start 184.9755 108.86186) (end 188.4934 112.37976) (width 0.25) (layer F.Cu) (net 15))
 (segment (start 184.9755 104.5083) (end 184.9755 108.86186) (width 0.25) (layer F.Cu) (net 15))
 (segment (start 181.3179 100.8507) (end 184.9755 104.5083) (width 0.25) (layer F.Cu) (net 15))
 (segment (start 179.3494 99.5807) (end 181.6481 99.5807) (width 0.25) (layer F.Cu) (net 16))
 (segment (start 186.1947 106.58348) (end 188.4934 108.88218) (width 0.25) (layer F.Cu) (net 16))
 (segment (start 186.1947 104.1273) (end 186.1947 106.58348) (width 0.25) (layer F.Cu) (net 16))
 (segment (start 181.6481 99.5807) (end 186.1947 104.1273) (width 0.25) (layer F.Cu) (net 16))
 (segment (start 179.3494 98.3107) (end 181.96814 98.3107) (width 0.25) (layer F.Cu) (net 17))
 (segment (start 181.96814 98.3107) (end 188.4934 104.83596) (width 0.25) (layer F.Cu) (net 17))
 (segment (start 179.3494 97.0407) (end 182.6133 97.0407) (width 0.25) (layer F.Cu) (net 18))
 (segment (start 186.91098 101.33838) (end 188.4934 101.33838) (width 0.25) (layer F.Cu) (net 18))
 (segment (start 182.6133 97.0407) (end 186.91098 101.33838) (width 0.25) (layer F.Cu) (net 18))
 (segment (start 184.78754 89.662) (end 190.246 89.662) (width 0.25) (layer F.Cu) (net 1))
 (segment (start 181.356 89.79154) (end 184.658 89.79154) (width 0.25) (layer F.Cu) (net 1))
 (segment (start 184.658 89.79154) (end 184.78754 89.662) (width 0.25) (layer F.Cu) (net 1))
 (segment (start 178.74996 89.99982) (end 181.14772 89.99982) (width 0.25) (layer F.Cu) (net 1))
 (segment (start 181.14772 89.99982) (end 181.356 89.79154) (width 0.25) (layer F.Cu) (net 1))
 (segment (start 164.846 98.298) (end 170.30446 98.298) (width 0.25) (layer F.Cu) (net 8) (status C00000))
 (segment (start 170.30446 98.298) (end 170.31716 98.3107) (width 0.25) (layer F.Cu) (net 8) (status C00000))
 (segment (start 170.31716 98.3107) (end 174.1424 98.3107) (width 0.25) (layer F.Cu) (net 8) (status C00000)))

